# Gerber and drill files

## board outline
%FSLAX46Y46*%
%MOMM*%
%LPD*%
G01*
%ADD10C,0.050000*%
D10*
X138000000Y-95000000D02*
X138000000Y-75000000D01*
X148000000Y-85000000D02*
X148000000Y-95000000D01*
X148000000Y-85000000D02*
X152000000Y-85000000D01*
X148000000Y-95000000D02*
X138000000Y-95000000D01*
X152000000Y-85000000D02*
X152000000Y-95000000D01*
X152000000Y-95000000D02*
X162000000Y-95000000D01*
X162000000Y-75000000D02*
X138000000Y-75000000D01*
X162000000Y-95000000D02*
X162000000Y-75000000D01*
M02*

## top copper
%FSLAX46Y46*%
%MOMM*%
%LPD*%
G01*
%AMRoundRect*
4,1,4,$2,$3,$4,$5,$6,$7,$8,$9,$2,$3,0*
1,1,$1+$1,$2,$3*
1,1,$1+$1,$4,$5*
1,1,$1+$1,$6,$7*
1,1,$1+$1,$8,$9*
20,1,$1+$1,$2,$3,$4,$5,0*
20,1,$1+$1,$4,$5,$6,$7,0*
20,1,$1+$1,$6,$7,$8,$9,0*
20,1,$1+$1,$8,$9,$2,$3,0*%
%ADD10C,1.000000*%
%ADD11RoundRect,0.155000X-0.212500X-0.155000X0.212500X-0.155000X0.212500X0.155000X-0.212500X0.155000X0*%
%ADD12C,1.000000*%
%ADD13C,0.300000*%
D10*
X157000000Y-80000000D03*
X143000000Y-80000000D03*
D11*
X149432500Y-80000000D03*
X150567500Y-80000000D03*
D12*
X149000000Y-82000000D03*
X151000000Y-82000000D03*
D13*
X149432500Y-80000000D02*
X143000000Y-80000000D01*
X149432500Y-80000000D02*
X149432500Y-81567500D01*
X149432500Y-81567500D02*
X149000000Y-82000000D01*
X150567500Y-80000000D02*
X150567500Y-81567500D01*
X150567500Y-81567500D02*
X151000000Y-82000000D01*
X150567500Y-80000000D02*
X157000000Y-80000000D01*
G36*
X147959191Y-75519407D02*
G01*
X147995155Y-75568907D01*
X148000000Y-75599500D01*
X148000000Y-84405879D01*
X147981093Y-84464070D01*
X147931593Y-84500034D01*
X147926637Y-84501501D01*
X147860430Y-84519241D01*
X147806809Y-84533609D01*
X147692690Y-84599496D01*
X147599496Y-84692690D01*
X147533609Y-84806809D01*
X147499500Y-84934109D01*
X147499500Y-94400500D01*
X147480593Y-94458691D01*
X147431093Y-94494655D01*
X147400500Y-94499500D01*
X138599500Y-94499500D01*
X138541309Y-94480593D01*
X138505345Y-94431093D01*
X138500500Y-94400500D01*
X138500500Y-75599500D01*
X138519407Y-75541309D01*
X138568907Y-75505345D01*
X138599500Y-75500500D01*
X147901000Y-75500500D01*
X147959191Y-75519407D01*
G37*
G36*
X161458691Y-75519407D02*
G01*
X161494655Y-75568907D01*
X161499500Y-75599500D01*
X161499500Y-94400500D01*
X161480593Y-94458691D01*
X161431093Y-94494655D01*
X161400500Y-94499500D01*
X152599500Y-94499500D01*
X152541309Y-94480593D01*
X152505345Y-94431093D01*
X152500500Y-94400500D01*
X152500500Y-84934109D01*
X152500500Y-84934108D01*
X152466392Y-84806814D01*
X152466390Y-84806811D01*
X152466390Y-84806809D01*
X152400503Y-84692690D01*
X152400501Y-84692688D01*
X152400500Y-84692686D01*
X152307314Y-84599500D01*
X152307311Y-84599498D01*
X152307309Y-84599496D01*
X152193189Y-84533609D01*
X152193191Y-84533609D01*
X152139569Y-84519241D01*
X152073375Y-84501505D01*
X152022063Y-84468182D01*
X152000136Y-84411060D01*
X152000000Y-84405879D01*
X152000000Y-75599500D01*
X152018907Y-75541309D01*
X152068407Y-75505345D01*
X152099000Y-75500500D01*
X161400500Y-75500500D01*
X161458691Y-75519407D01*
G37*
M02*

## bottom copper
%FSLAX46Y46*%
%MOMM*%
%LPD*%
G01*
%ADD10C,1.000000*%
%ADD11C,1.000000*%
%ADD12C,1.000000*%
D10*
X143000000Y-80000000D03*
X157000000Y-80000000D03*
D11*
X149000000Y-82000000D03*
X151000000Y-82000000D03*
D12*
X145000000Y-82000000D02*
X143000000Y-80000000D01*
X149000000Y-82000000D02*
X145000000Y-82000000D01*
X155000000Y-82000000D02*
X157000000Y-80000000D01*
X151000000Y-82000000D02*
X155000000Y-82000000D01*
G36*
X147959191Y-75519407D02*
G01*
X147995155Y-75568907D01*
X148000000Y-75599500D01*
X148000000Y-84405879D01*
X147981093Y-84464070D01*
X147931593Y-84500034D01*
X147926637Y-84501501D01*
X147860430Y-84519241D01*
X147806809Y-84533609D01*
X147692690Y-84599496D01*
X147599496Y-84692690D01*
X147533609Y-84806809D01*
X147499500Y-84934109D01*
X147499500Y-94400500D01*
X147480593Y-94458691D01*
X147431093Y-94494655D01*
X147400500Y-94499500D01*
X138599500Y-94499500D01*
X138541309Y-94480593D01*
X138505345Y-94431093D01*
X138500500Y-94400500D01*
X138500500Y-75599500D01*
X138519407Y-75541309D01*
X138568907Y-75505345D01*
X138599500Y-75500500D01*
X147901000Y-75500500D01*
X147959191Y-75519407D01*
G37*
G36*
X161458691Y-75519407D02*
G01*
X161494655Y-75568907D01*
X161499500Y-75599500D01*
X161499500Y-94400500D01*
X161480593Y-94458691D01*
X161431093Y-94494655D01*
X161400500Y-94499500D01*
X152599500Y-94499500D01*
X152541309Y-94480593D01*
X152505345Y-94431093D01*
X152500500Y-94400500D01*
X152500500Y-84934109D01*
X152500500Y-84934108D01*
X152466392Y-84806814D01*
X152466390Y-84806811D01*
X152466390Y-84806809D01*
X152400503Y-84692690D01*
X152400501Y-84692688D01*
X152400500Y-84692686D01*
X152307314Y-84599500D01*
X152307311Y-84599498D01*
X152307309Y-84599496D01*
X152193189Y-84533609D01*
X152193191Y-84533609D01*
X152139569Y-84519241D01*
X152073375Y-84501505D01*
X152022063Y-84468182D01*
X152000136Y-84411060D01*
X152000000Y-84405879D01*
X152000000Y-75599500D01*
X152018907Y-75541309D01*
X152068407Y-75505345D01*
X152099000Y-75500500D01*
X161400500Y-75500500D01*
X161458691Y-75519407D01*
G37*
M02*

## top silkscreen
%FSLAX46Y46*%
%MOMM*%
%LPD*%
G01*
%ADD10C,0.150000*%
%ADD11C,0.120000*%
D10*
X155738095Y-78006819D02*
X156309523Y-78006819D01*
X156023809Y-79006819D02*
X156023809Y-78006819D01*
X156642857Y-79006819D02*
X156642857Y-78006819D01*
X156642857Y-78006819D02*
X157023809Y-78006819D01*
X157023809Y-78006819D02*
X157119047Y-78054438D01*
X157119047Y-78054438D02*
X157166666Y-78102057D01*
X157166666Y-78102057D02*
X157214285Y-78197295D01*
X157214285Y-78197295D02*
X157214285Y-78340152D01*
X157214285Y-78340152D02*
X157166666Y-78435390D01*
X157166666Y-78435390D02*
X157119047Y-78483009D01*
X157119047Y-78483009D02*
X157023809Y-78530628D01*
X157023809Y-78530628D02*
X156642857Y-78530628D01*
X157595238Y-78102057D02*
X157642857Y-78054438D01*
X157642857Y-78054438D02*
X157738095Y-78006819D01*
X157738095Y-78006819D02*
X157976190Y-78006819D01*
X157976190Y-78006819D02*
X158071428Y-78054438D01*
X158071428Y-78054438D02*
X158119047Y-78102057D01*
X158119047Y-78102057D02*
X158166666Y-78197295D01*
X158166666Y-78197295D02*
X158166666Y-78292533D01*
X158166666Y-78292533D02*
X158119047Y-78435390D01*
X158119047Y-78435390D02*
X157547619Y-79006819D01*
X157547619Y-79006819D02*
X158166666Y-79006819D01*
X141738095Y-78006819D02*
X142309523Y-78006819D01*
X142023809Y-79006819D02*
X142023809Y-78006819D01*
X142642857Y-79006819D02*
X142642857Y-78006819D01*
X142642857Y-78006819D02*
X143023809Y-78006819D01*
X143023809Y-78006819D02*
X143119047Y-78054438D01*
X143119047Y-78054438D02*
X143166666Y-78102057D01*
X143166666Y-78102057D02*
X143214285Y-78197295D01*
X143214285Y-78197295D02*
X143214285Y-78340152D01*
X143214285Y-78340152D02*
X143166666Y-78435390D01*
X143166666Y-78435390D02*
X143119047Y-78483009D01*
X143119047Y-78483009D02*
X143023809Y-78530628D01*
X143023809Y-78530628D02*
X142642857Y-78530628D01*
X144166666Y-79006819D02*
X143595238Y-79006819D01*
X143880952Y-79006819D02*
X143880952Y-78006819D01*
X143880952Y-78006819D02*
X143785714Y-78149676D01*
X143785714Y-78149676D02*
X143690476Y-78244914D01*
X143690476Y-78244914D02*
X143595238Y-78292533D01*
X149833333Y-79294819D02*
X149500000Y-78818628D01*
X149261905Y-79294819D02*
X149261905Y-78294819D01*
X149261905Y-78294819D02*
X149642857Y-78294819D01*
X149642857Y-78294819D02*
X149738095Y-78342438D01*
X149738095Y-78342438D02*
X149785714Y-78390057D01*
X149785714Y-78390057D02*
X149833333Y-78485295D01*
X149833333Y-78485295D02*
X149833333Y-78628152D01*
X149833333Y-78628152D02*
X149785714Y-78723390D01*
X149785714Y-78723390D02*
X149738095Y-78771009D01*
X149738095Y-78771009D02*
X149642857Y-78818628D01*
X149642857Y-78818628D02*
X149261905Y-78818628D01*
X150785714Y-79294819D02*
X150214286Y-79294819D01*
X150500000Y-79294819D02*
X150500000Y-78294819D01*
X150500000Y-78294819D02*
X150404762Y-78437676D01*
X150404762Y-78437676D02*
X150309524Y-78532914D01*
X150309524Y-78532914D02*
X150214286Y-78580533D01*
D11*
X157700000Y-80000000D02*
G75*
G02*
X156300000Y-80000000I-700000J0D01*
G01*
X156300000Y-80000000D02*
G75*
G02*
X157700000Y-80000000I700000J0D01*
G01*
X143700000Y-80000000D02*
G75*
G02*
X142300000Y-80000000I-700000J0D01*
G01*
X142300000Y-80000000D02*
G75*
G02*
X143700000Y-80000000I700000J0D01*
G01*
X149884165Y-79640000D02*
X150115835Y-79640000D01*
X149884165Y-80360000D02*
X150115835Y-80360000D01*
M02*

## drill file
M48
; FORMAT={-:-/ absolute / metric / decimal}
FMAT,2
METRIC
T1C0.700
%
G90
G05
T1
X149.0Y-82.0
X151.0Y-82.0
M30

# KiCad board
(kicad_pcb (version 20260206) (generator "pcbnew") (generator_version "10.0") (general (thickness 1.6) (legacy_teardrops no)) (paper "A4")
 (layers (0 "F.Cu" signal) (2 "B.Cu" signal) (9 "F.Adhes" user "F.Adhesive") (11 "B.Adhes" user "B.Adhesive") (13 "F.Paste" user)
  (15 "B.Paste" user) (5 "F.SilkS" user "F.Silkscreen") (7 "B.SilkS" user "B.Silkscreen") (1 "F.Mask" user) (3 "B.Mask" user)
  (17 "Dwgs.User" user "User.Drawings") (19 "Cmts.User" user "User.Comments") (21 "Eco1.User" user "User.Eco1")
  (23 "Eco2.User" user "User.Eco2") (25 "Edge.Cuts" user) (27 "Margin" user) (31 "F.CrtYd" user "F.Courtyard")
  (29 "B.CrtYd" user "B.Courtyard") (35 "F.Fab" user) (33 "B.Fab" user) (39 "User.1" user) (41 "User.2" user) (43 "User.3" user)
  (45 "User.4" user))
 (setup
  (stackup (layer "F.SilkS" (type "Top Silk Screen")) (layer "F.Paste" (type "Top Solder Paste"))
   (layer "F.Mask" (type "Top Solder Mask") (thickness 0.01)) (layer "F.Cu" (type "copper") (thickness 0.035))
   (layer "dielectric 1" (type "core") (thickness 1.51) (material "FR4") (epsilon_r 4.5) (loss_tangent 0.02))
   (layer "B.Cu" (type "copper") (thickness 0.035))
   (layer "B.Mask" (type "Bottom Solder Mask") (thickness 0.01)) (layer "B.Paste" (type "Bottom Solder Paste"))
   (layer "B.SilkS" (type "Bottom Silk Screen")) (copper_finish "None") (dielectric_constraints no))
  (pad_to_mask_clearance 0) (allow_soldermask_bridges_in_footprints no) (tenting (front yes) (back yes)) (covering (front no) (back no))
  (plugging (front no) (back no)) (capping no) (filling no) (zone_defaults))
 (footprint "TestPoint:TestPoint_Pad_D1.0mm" (layer "F.Cu") (at 157 80)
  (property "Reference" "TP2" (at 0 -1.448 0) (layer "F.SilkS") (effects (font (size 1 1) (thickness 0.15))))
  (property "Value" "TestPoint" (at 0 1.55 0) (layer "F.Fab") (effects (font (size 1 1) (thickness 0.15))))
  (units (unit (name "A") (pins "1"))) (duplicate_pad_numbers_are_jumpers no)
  (fp_circle (center 0 0) (end 0 0.7) (stroke (width 0.12) (type solid)) (fill no) (layer "F.SilkS"))
  (pad "1" smd circle (at 0 0) (size 1 1) (layers "F.Cu" "F.Mask") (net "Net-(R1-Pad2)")))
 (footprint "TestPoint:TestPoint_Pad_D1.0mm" (layer "F.Cu") (at 143 80)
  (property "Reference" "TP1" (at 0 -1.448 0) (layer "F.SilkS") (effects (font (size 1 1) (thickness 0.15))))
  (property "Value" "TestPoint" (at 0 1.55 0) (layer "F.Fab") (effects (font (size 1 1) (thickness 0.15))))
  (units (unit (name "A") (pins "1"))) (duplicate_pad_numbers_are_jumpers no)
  (fp_circle (center 0 0) (end 0 0.7) (stroke (width 0.12) (type solid)) (fill no) (layer "F.SilkS"))
  (pad "1" smd circle (at 0 0) (size 1 1) (layers "F.Cu" "F.Mask") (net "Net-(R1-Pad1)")))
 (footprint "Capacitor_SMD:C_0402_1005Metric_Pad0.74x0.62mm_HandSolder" (layer "F.Cu") (at 150 80)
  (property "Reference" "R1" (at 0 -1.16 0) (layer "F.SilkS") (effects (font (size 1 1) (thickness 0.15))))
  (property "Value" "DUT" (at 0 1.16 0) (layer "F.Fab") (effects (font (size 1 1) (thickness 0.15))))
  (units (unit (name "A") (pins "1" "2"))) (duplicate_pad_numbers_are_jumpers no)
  (fp_line (start -0.115835 -0.36) (end 0.115835 -0.36) (stroke (width 0.12) (type solid)) (layer "F.SilkS"))
  (fp_line (start -0.115835 0.36) (end 0.115835 0.36) (stroke (width 0.12) (type solid)) (layer "F.SilkS"))
  (pad "1" smd roundrect (at -0.5675 0) (size 0.735 0.62) (layers "F.Cu" "F.Mask" "F.Paste") (roundrect_rratio 0.25) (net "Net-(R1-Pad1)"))
  (pad "2" smd roundrect (at 0.5675 0) (size 0.735 0.62) (layers "F.Cu" "F.Mask" "F.Paste") (roundrect_rratio 0.25) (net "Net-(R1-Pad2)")))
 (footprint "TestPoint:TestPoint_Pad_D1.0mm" (layer "B.Cu") (at 143 80 180)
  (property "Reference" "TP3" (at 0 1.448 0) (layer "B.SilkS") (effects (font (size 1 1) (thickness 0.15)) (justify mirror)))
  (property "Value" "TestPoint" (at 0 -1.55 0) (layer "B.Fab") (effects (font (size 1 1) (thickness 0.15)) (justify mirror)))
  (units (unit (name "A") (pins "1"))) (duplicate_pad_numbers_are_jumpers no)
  (pad "1" smd circle (at 0 0 180) (size 1 1) (layers "B.Cu" "B.Mask") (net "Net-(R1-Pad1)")))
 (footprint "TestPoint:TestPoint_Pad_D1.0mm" (layer "B.Cu") (at 157 80 180)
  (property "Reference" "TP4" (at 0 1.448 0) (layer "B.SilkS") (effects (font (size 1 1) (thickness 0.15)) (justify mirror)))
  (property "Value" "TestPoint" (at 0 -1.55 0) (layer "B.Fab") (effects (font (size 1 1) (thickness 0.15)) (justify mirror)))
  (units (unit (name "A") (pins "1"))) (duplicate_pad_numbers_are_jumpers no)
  (pad "1" smd circle (at 0 0 180) (size 1 1) (layers "B.Cu" "B.Mask") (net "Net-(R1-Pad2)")))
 (gr_line (start 138 95) (end 138 75) (stroke (width 0.05) (type default)) (layer "Edge.Cuts"))
 (gr_line (start 148 85) (end 148 95) (stroke (width 0.05) (type default)) (layer "Edge.Cuts"))
 (gr_line (start 148 85) (end 152 85) (stroke (width 0.05) (type default)) (layer "Edge.Cuts"))
 (gr_line (start 148 95) (end 138 95) (stroke (width 0.05) (type default)) (layer "Edge.Cuts"))
 (gr_line (start 152 85) (end 152 95) (stroke (width 0.05) (type default)) (layer "Edge.Cuts"))
 (gr_line (start 152 95) (end 162 95) (stroke (width 0.05) (type default)) (layer "Edge.Cuts"))
 (gr_line (start 162 75) (end 138 75) (stroke (width 0.05) (type default)) (layer "Edge.Cuts"))
 (gr_line (start 162 95) (end 162 75) (stroke (width 0.05) (type default)) (layer "Edge.Cuts"))
 (segment (start 149.4325 80) (end 143 80) (width 0.3) (layer "F.Cu") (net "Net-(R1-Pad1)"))
 (segment (start 149.4325 80) (end 149.4325 81.5675) (width 0.3) (layer "F.Cu") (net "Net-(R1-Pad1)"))
 (segment (start 149.4325 81.5675) (end 149 82) (width 0.3) (layer "F.Cu") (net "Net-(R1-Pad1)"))
 (via (at 149 82) (size 1) (drill 0.7) (layers "F.Cu" "B.Cu") (free yes) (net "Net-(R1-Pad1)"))
 (segment (start 145 82) (end 143 80) (width 1) (layer "B.Cu") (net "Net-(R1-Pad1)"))
 (segment (start 149 82) (end 145 82) (width 1) (layer "B.Cu") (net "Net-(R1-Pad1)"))
 (segment (start 150.5675 80) (end 150.5675 81.5675) (width 0.3) (layer "F.Cu") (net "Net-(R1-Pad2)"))
 (segment (start 150.5675 81.5675) (end 151 82) (width 0.3) (layer "F.Cu") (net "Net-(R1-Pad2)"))
 (segment (start 150.5675 80) (end 157 80) (width 0.3) (layer "F.Cu") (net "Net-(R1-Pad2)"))
 (via (at 151 82) (size 1) (drill 0.7) (layers "F.Cu" "B.Cu") (free yes) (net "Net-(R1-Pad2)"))
 (segment (start 155 82) (end 157 80) (width 1) (layer "B.Cu") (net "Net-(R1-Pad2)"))
 (segment (start 151 82) (end 155 82) (width 1) (layer "B.Cu") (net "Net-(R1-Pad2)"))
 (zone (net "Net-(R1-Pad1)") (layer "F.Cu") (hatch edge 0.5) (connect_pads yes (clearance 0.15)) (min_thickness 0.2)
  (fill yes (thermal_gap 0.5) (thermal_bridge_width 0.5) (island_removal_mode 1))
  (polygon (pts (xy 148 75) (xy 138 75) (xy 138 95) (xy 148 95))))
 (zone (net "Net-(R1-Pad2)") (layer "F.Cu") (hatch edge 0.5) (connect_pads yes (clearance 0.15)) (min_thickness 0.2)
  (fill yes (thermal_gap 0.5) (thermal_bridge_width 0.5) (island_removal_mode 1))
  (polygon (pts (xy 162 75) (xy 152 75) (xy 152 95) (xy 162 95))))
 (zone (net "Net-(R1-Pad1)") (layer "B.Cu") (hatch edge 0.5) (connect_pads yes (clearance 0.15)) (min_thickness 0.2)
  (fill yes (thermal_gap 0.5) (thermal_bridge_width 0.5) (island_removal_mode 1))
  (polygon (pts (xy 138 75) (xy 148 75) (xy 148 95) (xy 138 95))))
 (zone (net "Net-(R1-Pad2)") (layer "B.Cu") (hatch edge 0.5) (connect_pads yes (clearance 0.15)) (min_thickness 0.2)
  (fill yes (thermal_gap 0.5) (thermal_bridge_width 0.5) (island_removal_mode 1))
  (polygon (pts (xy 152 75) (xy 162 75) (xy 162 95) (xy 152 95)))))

